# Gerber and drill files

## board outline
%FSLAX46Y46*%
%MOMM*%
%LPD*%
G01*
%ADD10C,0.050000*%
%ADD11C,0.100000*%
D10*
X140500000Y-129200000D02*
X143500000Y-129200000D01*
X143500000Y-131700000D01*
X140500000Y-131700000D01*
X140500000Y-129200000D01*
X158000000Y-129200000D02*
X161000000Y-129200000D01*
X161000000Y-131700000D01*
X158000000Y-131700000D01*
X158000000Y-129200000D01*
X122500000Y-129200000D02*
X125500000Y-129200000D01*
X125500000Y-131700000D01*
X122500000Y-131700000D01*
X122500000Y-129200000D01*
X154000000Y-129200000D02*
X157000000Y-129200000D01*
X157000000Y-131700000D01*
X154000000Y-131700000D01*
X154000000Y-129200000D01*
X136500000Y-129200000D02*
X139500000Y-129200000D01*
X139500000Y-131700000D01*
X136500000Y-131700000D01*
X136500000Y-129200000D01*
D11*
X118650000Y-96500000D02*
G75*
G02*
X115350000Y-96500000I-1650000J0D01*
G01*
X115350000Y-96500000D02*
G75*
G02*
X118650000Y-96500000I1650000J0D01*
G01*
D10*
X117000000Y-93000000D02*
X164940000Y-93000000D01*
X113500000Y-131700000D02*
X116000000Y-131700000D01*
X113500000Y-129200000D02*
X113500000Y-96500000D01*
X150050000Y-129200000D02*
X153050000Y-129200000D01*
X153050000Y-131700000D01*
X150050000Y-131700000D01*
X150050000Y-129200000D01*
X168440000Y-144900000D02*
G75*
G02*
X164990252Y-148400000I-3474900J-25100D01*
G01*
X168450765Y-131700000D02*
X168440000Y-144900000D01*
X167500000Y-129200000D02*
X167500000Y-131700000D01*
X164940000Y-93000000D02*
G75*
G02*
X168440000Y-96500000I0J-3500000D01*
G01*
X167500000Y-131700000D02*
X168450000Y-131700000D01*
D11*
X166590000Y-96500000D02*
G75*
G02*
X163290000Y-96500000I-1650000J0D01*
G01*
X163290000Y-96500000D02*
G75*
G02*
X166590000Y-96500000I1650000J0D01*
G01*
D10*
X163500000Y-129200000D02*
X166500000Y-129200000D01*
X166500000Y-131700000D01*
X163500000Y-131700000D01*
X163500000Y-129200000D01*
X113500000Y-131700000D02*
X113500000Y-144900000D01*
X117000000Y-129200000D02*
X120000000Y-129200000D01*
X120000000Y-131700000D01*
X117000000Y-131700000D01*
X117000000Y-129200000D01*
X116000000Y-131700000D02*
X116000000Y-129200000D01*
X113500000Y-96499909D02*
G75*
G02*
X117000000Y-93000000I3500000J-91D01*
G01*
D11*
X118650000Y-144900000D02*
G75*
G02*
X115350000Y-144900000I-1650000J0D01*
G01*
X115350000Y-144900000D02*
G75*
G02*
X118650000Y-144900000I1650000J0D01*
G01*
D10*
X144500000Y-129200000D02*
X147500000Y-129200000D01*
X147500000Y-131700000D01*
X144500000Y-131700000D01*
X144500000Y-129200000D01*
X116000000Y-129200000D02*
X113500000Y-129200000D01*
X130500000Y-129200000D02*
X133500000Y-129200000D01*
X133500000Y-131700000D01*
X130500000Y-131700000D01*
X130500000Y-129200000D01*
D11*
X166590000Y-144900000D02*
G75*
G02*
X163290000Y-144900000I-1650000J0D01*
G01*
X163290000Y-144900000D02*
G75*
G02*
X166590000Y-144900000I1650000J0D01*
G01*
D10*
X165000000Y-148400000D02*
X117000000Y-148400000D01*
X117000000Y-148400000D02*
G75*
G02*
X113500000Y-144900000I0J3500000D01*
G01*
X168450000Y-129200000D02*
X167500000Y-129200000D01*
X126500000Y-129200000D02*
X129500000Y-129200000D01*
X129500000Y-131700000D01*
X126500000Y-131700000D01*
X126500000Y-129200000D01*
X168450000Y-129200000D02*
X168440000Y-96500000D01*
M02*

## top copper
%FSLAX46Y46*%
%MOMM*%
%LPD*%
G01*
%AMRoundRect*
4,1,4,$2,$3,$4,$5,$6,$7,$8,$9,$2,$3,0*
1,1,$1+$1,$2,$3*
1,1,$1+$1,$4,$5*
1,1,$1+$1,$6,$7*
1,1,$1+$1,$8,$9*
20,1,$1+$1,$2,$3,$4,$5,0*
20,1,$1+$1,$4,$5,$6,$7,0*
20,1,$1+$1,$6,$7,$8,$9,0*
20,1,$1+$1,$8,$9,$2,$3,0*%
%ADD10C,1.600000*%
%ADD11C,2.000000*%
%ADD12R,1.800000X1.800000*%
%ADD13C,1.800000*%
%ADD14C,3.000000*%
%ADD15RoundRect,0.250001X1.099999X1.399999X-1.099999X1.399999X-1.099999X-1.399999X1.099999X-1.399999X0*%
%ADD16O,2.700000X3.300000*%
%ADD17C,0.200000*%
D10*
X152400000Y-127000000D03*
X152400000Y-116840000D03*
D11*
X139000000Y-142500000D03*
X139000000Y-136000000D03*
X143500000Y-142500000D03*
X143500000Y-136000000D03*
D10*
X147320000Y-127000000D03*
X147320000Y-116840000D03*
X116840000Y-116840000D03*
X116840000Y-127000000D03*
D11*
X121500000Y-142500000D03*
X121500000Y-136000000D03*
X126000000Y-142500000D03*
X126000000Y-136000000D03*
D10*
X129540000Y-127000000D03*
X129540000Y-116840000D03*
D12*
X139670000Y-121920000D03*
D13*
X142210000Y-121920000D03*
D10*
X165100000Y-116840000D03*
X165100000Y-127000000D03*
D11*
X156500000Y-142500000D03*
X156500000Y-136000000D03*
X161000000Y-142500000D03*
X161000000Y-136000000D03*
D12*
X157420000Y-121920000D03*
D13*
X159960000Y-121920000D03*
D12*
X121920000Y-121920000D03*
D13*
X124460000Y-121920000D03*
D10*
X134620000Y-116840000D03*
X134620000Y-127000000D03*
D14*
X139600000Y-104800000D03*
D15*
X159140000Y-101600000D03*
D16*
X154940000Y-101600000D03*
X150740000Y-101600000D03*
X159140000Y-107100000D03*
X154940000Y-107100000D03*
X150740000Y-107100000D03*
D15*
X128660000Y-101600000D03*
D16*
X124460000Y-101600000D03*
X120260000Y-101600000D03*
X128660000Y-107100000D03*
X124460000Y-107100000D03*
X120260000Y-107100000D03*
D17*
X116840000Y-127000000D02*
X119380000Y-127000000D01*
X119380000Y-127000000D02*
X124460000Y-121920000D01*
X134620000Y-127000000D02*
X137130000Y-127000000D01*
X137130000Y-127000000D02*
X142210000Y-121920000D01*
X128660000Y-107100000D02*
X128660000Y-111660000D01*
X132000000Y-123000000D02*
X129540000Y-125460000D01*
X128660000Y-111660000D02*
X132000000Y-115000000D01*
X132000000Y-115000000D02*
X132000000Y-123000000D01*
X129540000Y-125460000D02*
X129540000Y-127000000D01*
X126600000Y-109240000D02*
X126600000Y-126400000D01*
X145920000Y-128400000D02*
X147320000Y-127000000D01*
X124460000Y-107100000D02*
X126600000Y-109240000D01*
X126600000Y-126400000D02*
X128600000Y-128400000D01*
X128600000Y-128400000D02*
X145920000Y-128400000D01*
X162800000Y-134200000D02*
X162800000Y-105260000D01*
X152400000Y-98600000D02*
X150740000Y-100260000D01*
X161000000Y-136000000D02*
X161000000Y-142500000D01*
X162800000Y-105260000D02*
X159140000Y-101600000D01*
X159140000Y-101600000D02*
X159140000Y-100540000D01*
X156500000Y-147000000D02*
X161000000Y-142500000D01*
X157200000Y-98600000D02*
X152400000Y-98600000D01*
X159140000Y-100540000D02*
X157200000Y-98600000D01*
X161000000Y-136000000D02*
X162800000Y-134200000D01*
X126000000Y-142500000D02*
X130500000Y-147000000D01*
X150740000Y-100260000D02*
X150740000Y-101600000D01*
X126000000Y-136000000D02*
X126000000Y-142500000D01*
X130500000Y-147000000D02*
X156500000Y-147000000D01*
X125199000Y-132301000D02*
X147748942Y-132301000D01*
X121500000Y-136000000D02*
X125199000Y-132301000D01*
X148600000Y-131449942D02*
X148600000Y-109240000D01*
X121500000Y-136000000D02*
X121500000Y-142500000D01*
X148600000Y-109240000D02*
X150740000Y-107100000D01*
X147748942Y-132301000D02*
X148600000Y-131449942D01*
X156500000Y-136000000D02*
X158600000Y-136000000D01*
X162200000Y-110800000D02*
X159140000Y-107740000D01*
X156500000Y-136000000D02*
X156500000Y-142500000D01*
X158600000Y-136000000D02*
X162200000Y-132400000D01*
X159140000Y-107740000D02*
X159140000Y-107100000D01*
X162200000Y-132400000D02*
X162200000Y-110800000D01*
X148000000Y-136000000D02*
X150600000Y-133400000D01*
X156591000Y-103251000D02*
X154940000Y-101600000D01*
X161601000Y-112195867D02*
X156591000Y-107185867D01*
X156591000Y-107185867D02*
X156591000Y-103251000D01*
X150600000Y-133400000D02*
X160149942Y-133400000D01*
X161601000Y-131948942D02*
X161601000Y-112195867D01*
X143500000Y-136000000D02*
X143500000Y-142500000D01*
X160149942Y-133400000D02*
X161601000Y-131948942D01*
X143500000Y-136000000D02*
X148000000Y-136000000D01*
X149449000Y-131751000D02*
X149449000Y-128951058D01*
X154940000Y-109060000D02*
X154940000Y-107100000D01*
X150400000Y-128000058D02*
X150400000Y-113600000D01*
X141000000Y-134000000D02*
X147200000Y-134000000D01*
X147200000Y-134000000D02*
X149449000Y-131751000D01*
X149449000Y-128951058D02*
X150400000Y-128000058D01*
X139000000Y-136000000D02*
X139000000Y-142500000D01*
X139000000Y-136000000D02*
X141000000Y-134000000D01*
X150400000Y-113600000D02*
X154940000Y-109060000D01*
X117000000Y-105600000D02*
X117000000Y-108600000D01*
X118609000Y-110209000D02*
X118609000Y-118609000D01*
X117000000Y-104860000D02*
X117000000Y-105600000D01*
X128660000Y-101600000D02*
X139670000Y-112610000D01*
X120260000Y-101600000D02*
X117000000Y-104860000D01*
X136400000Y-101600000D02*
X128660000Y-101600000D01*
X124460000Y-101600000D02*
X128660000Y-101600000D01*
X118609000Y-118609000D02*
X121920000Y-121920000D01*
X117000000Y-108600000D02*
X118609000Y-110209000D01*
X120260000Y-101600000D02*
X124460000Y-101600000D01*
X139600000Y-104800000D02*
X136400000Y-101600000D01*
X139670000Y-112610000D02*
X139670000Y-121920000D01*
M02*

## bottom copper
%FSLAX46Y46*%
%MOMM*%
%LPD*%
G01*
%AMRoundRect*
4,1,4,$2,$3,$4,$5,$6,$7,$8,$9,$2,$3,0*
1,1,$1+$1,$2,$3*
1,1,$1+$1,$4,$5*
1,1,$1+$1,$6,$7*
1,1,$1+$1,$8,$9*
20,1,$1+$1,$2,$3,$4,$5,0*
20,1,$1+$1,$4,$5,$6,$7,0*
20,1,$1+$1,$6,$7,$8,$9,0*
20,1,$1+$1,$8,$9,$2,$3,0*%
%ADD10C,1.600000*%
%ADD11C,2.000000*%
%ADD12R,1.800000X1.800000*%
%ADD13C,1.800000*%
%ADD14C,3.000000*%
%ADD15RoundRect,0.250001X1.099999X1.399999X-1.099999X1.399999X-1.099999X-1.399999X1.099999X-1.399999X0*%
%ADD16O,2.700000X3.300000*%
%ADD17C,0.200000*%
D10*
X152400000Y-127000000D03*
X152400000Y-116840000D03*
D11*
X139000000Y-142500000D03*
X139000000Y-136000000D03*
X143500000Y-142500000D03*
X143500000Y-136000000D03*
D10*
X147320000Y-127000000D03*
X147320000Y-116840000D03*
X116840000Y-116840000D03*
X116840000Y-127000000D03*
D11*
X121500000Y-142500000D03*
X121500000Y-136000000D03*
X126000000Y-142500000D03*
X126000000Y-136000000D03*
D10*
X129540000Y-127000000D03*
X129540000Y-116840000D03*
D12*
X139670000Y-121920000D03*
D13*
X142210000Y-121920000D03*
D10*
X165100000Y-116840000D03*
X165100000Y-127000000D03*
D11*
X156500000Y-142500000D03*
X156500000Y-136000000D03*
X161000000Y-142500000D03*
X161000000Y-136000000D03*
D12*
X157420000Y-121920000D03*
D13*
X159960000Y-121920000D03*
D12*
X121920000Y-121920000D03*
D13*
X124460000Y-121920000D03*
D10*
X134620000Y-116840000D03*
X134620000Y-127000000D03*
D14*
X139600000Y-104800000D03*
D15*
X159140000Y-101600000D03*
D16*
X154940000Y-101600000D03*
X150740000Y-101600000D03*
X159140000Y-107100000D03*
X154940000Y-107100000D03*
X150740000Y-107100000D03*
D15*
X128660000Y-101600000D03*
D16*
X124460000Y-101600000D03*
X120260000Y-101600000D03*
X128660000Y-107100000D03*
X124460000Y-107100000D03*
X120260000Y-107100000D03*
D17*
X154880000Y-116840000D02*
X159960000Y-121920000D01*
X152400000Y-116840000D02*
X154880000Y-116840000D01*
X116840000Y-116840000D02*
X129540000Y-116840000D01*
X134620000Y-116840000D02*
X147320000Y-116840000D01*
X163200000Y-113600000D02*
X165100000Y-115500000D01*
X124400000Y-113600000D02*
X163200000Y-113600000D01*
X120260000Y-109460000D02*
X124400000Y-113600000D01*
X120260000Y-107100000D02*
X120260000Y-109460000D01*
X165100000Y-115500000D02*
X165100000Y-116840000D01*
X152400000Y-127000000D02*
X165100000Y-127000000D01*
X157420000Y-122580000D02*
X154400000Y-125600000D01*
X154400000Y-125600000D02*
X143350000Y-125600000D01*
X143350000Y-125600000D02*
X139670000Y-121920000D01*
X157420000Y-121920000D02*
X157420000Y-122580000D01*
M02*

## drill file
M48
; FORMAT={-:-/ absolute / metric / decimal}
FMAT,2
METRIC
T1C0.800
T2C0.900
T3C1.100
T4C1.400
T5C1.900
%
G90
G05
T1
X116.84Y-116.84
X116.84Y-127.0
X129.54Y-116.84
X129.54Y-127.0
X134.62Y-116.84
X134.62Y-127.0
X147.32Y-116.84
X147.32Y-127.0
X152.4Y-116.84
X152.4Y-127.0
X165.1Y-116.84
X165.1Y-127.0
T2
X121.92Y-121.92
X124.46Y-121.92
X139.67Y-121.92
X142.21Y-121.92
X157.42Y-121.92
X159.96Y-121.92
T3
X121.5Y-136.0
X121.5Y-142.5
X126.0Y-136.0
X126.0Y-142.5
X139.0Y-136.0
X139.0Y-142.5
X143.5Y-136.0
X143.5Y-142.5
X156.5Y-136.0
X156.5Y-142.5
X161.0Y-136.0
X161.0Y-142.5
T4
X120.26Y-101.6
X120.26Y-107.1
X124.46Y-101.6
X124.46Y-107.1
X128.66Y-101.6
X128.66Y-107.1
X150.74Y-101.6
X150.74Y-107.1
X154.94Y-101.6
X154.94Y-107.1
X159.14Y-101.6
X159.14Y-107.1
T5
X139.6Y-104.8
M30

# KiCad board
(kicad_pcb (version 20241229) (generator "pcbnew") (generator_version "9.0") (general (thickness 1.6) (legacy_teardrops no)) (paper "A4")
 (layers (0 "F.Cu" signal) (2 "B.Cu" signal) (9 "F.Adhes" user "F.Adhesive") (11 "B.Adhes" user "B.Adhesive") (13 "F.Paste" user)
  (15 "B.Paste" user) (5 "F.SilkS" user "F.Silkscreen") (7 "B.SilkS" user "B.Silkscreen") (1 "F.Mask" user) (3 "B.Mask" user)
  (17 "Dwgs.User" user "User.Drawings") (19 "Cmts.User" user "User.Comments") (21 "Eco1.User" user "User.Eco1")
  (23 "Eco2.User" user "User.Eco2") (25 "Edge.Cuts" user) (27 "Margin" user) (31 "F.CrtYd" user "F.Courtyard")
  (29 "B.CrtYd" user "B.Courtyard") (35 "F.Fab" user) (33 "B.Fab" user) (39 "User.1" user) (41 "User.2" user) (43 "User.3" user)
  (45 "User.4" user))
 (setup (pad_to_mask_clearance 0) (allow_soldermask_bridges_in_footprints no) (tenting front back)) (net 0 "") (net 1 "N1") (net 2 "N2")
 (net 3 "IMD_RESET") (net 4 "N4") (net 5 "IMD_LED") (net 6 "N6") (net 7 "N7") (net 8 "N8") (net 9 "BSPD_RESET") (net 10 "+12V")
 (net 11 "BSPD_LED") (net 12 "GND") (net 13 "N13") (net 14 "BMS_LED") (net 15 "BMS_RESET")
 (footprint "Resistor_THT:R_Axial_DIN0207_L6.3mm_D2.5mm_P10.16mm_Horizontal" (layer "F.Cu") (at 152.4 127 90)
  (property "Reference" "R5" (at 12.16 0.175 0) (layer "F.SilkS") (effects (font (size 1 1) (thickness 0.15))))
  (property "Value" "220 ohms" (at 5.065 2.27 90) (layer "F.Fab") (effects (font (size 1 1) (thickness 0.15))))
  (pad "1" thru_hole circle (at 0 0 90) (size 1.6 1.6) (drill 0.8) (layers "*.Cu" "*.Mask") (remove_unused_layers no) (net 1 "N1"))
  (pad "2" thru_hole circle (at 10.16 0 90) (size 1.6 1.6) (drill 0.8) (layers "*.Cu" "*.Mask") (remove_unused_layers no) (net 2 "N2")))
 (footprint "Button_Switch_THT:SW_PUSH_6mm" (layer "F.Cu") (at 139 142.5 90)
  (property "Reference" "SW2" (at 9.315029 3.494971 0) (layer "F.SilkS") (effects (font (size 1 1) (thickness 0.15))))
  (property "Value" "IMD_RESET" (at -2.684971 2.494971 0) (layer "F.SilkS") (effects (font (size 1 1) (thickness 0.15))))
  (pad "1" thru_hole circle (at 0 0 180) (size 2 2) (drill 1.1) (layers "*.Cu" "*.Mask") (remove_unused_layers no) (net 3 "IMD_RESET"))
  (pad "1" thru_hole circle (at 6.5 0 180) (size 2 2) (drill 1.1) (layers "*.Cu" "*.Mask") (remove_unused_layers no) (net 3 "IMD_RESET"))
  (pad "2" thru_hole circle (at 0 4.5 180) (size 2 2) (drill 1.1) (layers "*.Cu" "*.Mask") (remove_unused_layers no) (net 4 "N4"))
  (pad "2" thru_hole circle (at 6.5 4.5 180) (size 2 2) (drill 1.1) (layers "*.Cu" "*.Mask") (remove_unused_layers no) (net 4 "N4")))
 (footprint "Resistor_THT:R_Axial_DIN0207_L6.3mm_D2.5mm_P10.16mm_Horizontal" (layer "F.Cu") (at 147.32 127 90)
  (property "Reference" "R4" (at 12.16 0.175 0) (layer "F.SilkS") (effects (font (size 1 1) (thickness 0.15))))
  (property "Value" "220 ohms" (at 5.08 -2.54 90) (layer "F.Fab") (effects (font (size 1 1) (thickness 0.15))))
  (pad "1" thru_hole circle (at 0 0 90) (size 1.6 1.6) (drill 0.8) (layers "*.Cu" "*.Mask") (remove_unused_layers no) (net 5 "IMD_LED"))
  (pad "2" thru_hole circle (at 10.16 0 90) (size 1.6 1.6) (drill 0.8) (layers "*.Cu" "*.Mask") (remove_unused_layers no) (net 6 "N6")))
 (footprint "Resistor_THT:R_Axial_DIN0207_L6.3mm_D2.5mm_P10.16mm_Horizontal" (layer "F.Cu") (at 116.84 116.84 -90)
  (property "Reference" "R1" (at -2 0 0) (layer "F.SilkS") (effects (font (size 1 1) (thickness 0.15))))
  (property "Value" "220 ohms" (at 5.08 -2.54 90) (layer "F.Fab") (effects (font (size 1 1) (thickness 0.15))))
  (pad "1" thru_hole circle (at 0 0 270) (size 1.6 1.6) (drill 0.8) (layers "*.Cu" "*.Mask") (remove_unused_layers no) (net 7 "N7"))
  (pad "2" thru_hole circle (at 10.16 0 270) (size 1.6 1.6) (drill 0.8) (layers "*.Cu" "*.Mask") (remove_unused_layers no) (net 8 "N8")))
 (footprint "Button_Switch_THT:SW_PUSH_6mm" (layer "F.Cu") (at 121.5 142.5 90)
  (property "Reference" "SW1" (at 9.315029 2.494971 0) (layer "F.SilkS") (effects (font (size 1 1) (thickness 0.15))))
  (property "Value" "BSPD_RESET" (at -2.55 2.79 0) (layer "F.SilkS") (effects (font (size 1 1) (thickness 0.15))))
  (pad "1" thru_hole circle (at 0 0 180) (size 2 2) (drill 1.1) (layers "*.Cu" "*.Mask") (remove_unused_layers no) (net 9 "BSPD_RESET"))
  (pad "1" thru_hole circle (at 6.5 0 180) (size 2 2) (drill 1.1) (layers "*.Cu" "*.Mask") (remove_unused_layers no) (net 9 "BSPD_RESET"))
  (pad "2" thru_hole circle (at 0 4.5 180) (size 2 2) (drill 1.1) (layers "*.Cu" "*.Mask") (remove_unused_layers no) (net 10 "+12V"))
  (pad "2" thru_hole circle (at 6.5 4.5 180) (size 2 2) (drill 1.1) (layers "*.Cu" "*.Mask") (remove_unused_layers no) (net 10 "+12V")))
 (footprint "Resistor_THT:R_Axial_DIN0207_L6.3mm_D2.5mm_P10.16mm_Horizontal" (layer "F.Cu") (at 129.54 127 90)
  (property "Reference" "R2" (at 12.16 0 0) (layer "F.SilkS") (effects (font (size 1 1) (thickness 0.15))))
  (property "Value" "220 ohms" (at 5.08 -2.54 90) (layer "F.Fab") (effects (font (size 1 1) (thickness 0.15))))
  (pad "1" thru_hole circle (at 0 0 90) (size 1.6 1.6) (drill 0.8) (layers "*.Cu" "*.Mask") (remove_unused_layers no) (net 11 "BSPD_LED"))
  (pad "2" thru_hole circle (at 10.16 0 90) (size 1.6 1.6) (drill 0.8) (layers "*.Cu" "*.Mask") (remove_unused_layers no) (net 7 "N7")))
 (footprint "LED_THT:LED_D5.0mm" (layer "F.Cu") (at 139.67 121.92)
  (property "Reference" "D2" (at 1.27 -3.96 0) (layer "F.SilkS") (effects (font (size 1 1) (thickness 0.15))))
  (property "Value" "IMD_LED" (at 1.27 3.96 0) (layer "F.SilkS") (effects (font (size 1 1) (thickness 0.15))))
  (pad "1" thru_hole rect (at 0 0) (size 1.8 1.8) (drill 0.9) (layers "*.Cu" "*.Mask") (remove_unused_layers no) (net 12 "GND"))
  (pad "2" thru_hole circle (at 2.54 0) (size 1.8 1.8) (drill 0.9) (layers "*.Cu" "*.Mask") (remove_unused_layers no) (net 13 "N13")))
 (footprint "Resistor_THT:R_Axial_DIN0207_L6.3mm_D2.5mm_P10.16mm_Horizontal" (layer "F.Cu") (at 165.1 116.84 -90)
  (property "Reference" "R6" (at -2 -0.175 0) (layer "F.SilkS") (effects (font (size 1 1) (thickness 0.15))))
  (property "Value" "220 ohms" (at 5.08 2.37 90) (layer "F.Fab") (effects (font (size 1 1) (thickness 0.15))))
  (pad "1" thru_hole circle (at 0 0 270) (size 1.6 1.6) (drill 0.8) (layers "*.Cu" "*.Mask") (remove_unused_layers no) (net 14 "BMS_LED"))
  (pad "2" thru_hole circle (at 10.16 0 270) (size 1.6 1.6) (drill 0.8) (layers "*.Cu" "*.Mask") (remove_unused_layers no) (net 1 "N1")))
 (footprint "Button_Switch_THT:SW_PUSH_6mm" (layer "F.Cu") (at 156.5 142.5 90)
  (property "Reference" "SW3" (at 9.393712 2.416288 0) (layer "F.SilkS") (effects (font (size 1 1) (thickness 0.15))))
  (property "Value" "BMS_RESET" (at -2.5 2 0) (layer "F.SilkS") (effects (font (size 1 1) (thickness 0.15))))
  (pad "1" thru_hole circle (at 0 0 180) (size 2 2) (drill 1.1) (layers "*.Cu" "*.Mask") (remove_unused_layers no) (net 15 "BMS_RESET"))
  (pad "1" thru_hole circle (at 6.5 0 180) (size 2 2) (drill 1.1) (layers "*.Cu" "*.Mask") (remove_unused_layers no) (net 15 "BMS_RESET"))
  (pad "2" thru_hole circle (at 0 4.5 180) (size 2 2) (drill 1.1) (layers "*.Cu" "*.Mask") (remove_unused_layers no) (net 10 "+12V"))
  (pad "2" thru_hole circle (at 6.5 4.5 180) (size 2 2) (drill 1.1) (layers "*.Cu" "*.Mask") (remove_unused_layers no) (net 10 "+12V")))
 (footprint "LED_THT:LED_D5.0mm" (layer "F.Cu") (at 157.42 121.92)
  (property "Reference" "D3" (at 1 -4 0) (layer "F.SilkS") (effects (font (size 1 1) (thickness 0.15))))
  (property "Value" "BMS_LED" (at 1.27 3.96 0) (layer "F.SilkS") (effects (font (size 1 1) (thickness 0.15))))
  (pad "1" thru_hole rect (at 0 0) (size 1.8 1.8) (drill 0.9) (layers "*.Cu" "*.Mask") (remove_unused_layers no) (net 12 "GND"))
  (pad "2" thru_hole circle (at 2.54 0) (size 1.8 1.8) (drill 0.9) (layers "*.Cu" "*.Mask") (remove_unused_layers no) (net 2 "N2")))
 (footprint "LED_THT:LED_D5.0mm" (layer "F.Cu") (at 121.92 121.92)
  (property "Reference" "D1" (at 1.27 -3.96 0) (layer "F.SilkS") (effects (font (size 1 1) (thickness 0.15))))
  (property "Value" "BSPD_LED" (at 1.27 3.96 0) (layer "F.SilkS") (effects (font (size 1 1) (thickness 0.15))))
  (pad "1" thru_hole rect (at 0 0) (size 1.8 1.8) (drill 0.9) (layers "*.Cu" "*.Mask") (remove_unused_layers no) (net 12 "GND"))
  (pad "2" thru_hole circle (at 2.54 0) (size 1.8 1.8) (drill 0.9) (layers "*.Cu" "*.Mask") (remove_unused_layers no) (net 8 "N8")))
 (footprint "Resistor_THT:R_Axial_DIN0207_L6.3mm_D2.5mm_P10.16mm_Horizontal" (layer "F.Cu") (at 134.62 116.84 -90)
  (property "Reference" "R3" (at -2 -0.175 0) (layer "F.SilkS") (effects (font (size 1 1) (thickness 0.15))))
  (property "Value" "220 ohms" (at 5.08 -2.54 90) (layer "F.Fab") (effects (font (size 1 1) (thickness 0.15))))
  (pad "1" thru_hole circle (at 0 0 270) (size 1.6 1.6) (drill 0.8) (layers "*.Cu" "*.Mask") (remove_unused_layers no) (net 6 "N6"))
  (pad "2" thru_hole circle (at 10.16 0 270) (size 1.6 1.6) (drill 0.8) (layers "*.Cu" "*.Mask") (remove_unused_layers no) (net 13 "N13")))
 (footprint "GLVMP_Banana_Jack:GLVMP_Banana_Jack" (layer "B.Cu") (at 139.6 104.8 180)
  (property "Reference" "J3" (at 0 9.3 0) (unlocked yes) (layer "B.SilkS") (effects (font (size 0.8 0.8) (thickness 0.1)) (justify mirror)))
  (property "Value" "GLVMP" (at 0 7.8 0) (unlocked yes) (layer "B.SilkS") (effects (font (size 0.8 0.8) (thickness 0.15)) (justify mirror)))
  (pad "1" thru_hole circle (at 0 0 180) (size 3 3) (drill 1.9) (layers "*.Cu" "*.Mask") (remove_unused_layers no) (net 12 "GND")))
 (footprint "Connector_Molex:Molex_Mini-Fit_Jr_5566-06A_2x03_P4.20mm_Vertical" (layer "B.Cu") (at 159.14 101.6 180)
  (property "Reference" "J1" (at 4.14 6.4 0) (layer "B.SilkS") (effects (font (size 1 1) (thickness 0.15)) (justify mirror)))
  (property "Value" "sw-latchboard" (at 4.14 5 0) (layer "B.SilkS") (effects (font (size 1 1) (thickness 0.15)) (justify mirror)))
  (pad "1" thru_hole roundrect (at 0 0 180) (size 2.7 3.3) (drill 1.4) (layers "*.Cu" "*.Mask") (remove_unused_layers no)
   (roundrect_rratio 0.092593) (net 10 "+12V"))
  (pad "2" thru_hole oval (at 4.2 0 180) (size 2.7 3.3) (drill 1.4) (layers "*.Cu" "*.Mask") (remove_unused_layers no) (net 4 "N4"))
  (pad "3" thru_hole oval (at 8.4 0 180) (size 2.7 3.3) (drill 1.4) (layers "*.Cu" "*.Mask") (remove_unused_layers no) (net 10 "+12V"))
  (pad "4" thru_hole oval (at 0 -5.5 180) (size 2.7 3.3) (drill 1.4) (layers "*.Cu" "*.Mask") (remove_unused_layers no) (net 15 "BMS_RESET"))
  (pad "5" thru_hole oval (at 4.2 -5.5 180) (size 2.7 3.3) (drill 1.4) (layers "*.Cu" "*.Mask") (remove_unused_layers no)
   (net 3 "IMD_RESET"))
  (pad "6" thru_hole oval (at 8.4 -5.5 180) (size 2.7 3.3) (drill 1.4) (layers "*.Cu" "*.Mask") (remove_unused_layers no)
   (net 9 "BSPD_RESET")))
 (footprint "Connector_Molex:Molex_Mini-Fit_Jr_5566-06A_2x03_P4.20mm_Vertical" (layer "B.Cu") (at 128.66 101.6 180)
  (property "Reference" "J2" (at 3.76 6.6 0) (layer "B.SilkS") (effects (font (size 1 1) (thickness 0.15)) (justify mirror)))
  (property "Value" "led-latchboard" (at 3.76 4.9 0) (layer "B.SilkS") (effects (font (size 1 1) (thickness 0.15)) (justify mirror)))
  (pad "1" thru_hole roundrect (at 0 0 180) (size 2.7 3.3) (drill 1.4) (layers "*.Cu" "*.Mask") (remove_unused_layers no)
   (roundrect_rratio 0.092593) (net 12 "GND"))
  (pad "2" thru_hole oval (at 4.2 0 180) (size 2.7 3.3) (drill 1.4) (layers "*.Cu" "*.Mask") (remove_unused_layers no) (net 12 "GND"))
  (pad "3" thru_hole oval (at 8.4 0 180) (size 2.7 3.3) (drill 1.4) (layers "*.Cu" "*.Mask") (remove_unused_layers no) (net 12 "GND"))
  (pad "4" thru_hole oval (at 0 -5.5 180) (size 2.7 3.3) (drill 1.4) (layers "*.Cu" "*.Mask") (remove_unused_layers no) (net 11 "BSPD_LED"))
  (pad "5" thru_hole oval (at 4.2 -5.5 180) (size 2.7 3.3) (drill 1.4) (layers "*.Cu" "*.Mask") (remove_unused_layers no) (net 5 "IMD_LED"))
  (pad "6" thru_hole oval (at 8.4 -5.5 180) (size 2.7 3.3) (drill 1.4) (layers "*.Cu" "*.Mask") (remove_unused_layers no) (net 14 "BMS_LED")))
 (gr_rect (start 140.5 129.2) (end 143.5 131.7) (stroke (width 0.05) (type default)) (fill no) (layer "Edge.Cuts"))
 (gr_rect (start 158 129.2) (end 161 131.7) (stroke (width 0.05) (type default)) (fill no) (layer "Edge.Cuts"))
 (gr_rect (start 122.5 129.2) (end 125.5 131.7) (stroke (width 0.05) (type default)) (fill no) (layer "Edge.Cuts"))
 (gr_rect (start 154 129.2) (end 157 131.7) (stroke (width 0.05) (type default)) (fill no) (layer "Edge.Cuts"))
 (gr_rect (start 136.5 129.2) (end 139.5 131.7) (stroke (width 0.05) (type default)) (fill no) (layer "Edge.Cuts"))
 (gr_circle (center 117 96.5) (end 118.65 96.5) (stroke (width 0.1) (type solid)) (fill no) (layer "Edge.Cuts"))
 (gr_line (start 117 93) (end 164.94 93) (stroke (width 0.05) (type default)) (layer "Edge.Cuts"))
 (gr_line (start 113.5 131.7) (end 116 131.7) (stroke (width 0.05) (type default)) (layer "Edge.Cuts"))
 (gr_line (start 113.5 129.2) (end 113.5 96.5) (stroke (width 0.05) (type default)) (layer "Edge.Cuts"))
 (gr_rect (start 150.05 129.2) (end 153.05 131.7) (stroke (width 0.05) (type default)) (fill no) (layer "Edge.Cuts"))
 (gr_arc (start 168.44 144.9) (mid 167.44 147.364466) (end 164.990252 148.4) (stroke (width 0.05) (type solid)) (layer "Edge.Cuts"))
 (gr_line (start 168.450765 131.7) (end 168.44 144.9) (stroke (width 0.05) (type default)) (layer "Edge.Cuts"))
 (gr_line (start 167.5 129.2) (end 167.5 131.7) (stroke (width 0.05) (type default)) (layer "Edge.Cuts"))
 (gr_arc (start 164.94 93) (mid 167.414874 94.025126) (end 168.44 96.5) (stroke (width 0.05) (type solid)) (layer "Edge.Cuts"))
 (gr_line (start 167.5 131.7) (end 168.45 131.7) (stroke (width 0.05) (type default)) (layer "Edge.Cuts"))
 (gr_circle (center 164.94 96.5) (end 166.59 96.5) (stroke (width 0.1) (type solid)) (fill no) (layer "Edge.Cuts"))
 (gr_rect (start 163.5 129.2) (end 166.5 131.7) (stroke (width 0.05) (type default)) (fill no) (layer "Edge.Cuts"))
 (gr_line (start 113.5 131.7) (end 113.5 144.9) (stroke (width 0.05) (type solid)) (layer "Edge.Cuts"))
 (gr_rect (start 117 129.2) (end 120 131.7) (stroke (width 0.05) (type default)) (fill no) (layer "Edge.Cuts"))
 (gr_line (start 116 131.7) (end 116 129.2) (stroke (width 0.05) (type default)) (layer "Edge.Cuts"))
 (gr_arc (start 113.5 96.499909) (mid 114.525158 94.025094) (end 117 93) (stroke (width 0.05) (type default)) (layer "Edge.Cuts"))
 (gr_circle (center 117 144.9) (end 115.35 144.9) (stroke (width 0.1) (type solid)) (fill no) (layer "Edge.Cuts"))
 (gr_rect (start 144.5 129.2) (end 147.5 131.7) (stroke (width 0.05) (type default)) (fill no) (layer "Edge.Cuts"))
 (gr_line (start 116 129.2) (end 113.5 129.2) (stroke (width 0.05) (type default)) (layer "Edge.Cuts"))
 (gr_rect (start 130.5 129.2) (end 133.5 131.7) (stroke (width 0.05) (type default)) (fill no) (layer "Edge.Cuts"))
 (gr_circle (center 164.94 144.9) (end 163.29 144.9) (stroke (width 0.1) (type solid)) (fill no) (layer "Edge.Cuts"))
 (gr_line (start 165 148.4) (end 117 148.4) (stroke (width 0.05) (type solid)) (layer "Edge.Cuts"))
 (gr_arc (start 117 148.4) (mid 114.525126 147.374874) (end 113.5 144.9) (stroke (width 0.05) (type solid)) (layer "Edge.Cuts"))
 (gr_line (start 168.45 129.2) (end 167.5 129.2) (stroke (width 0.05) (type default)) (layer "Edge.Cuts"))
 (gr_rect (start 126.5 129.2) (end 129.5 131.7) (stroke (width 0.05) (type default)) (fill no) (layer "Edge.Cuts"))
 (gr_line (start 168.45 129.2) (end 168.44 96.5) (stroke (width 0.05) (type default)) (layer "Edge.Cuts"))
 (segment (start 116.84 127) (end 119.38 127) (width 0.2) (layer "F.Cu") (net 8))
 (segment (start 119.38 127) (end 124.46 121.92) (width 0.2) (layer "F.Cu") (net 8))
 (segment (start 134.62 127) (end 137.13 127) (width 0.2) (layer "F.Cu") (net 13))
 (segment (start 137.13 127) (end 142.21 121.92) (width 0.2) (layer "F.Cu") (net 13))
 (segment (start 154.88 116.84) (end 159.96 121.92) (width 0.2) (layer "B.Cu") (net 2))
 (segment (start 152.4 116.84) (end 154.88 116.84) (width 0.2) (layer "B.Cu") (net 2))
 (segment (start 116.84 116.84) (end 129.54 116.84) (width 0.2) (layer "B.Cu") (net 7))
 (segment (start 128.66 107.1) (end 128.66 111.66) (width 0.2) (layer "F.Cu") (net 11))
 (segment (start 132 123) (end 129.54 125.46) (width 0.2) (layer "F.Cu") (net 11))
 (segment (start 128.66 111.66) (end 132 115) (width 0.2) (layer "F.Cu") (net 11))
 (segment (start 132 115) (end 132 123) (width 0.2) (layer "F.Cu") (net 11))
 (segment (start 129.54 125.46) (end 129.54 127) (width 0.2) (layer "F.Cu") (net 11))
 (segment (start 134.62 116.84) (end 147.32 116.84) (width 0.2) (layer "B.Cu") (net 6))
 (segment (start 126.6 109.24) (end 126.6 126.4) (width 0.2) (layer "F.Cu") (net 5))
 (segment (start 145.92 128.4) (end 147.32 127) (width 0.2) (layer "F.Cu") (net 5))
 (segment (start 124.46 107.1) (end 126.6 109.24) (width 0.2) (layer "F.Cu") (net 5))
 (segment (start 126.6 126.4) (end 128.6 128.4) (width 0.2) (layer "F.Cu") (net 5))
 (segment (start 128.6 128.4) (end 145.92 128.4) (width 0.2) (layer "F.Cu") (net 5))
 (segment (start 163.2 113.6) (end 165.1 115.5) (width 0.2) (layer "B.Cu") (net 14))
 (segment (start 124.4 113.6) (end 163.2 113.6) (width 0.2) (layer "B.Cu") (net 14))
 (segment (start 120.26 109.46) (end 124.4 113.6) (width 0.2) (layer "B.Cu") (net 14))
 (segment (start 120.26 107.1) (end 120.26 109.46) (width 0.2) (layer "B.Cu") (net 14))
 (segment (start 165.1 115.5) (end 165.1 116.84) (width 0.2) (layer "B.Cu") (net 14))
 (segment (start 162.8 134.2) (end 162.8 105.26) (width 0.2) (layer "F.Cu") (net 10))
 (segment (start 152.4 98.6) (end 150.74 100.26) (width 0.2) (layer "F.Cu") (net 10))
 (segment (start 161 136) (end 161 142.5) (width 0.2) (layer "F.Cu") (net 10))
 (segment (start 162.8 105.26) (end 159.14 101.6) (width 0.2) (layer "F.Cu") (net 10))
 (segment (start 159.14 101.6) (end 159.14 100.54) (width 0.2) (layer "F.Cu") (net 10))
 (segment (start 156.5 147) (end 161 142.5) (width 0.2) (layer "F.Cu") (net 10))
 (segment (start 157.2 98.6) (end 152.4 98.6) (width 0.2) (layer "F.Cu") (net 10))
 (segment (start 159.14 100.54) (end 157.2 98.6) (width 0.2) (layer "F.Cu") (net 10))
 (segment (start 161 136) (end 162.8 134.2) (width 0.2) (layer "F.Cu") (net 10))
 (segment (start 126 142.5) (end 130.5 147) (width 0.2) (layer "F.Cu") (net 10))
 (segment (start 150.74 100.26) (end 150.74 101.6) (width 0.2) (layer "F.Cu") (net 10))
 (segment (start 126 136) (end 126 142.5) (width 0.2) (layer "F.Cu") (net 10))
 (segment (start 130.5 147) (end 156.5 147) (width 0.2) (layer "F.Cu") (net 10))
 (segment (start 125.199 132.301) (end 147.748942 132.301) (width 0.2) (layer "F.Cu") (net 9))
 (segment (start 121.5 136) (end 125.199 132.301) (width 0.2) (layer "F.Cu") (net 9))
 (segment (start 148.6 131.449942) (end 148.6 109.24) (width 0.2) (layer "F.Cu") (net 9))
 (segment (start 121.5 136) (end 121.5 142.5) (width 0.2) (layer "F.Cu") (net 9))
 (segment (start 148.6 109.24) (end 150.74 107.1) (width 0.2) (layer "F.Cu") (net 9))
 (segment (start 147.748942 132.301) (end 148.6 131.449942) (width 0.2) (layer "F.Cu") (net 9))
 (segment (start 156.5 136) (end 158.6 136) (width 0.2) (layer "F.Cu") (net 15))
 (segment (start 162.2 110.8) (end 159.14 107.74) (width 0.2) (layer "F.Cu") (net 15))
 (segment (start 156.5 136) (end 156.5 142.5) (width 0.2) (layer "F.Cu") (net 15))
 (segment (start 158.6 136) (end 162.2 132.4) (width 0.2) (layer "F.Cu") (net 15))
 (segment (start 159.14 107.74) (end 159.14 107.1) (width 0.2) (layer "F.Cu") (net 15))
 (segment (start 162.2 132.4) (end 162.2 110.8) (width 0.2) (layer "F.Cu") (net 15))
 (segment (start 148 136) (end 150.6 133.4) (width 0.2) (layer "F.Cu") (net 4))
 (segment (start 156.591 103.251) (end 154.94 101.6) (width 0.2) (layer "F.Cu") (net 4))
 (segment (start 161.601 112.195867) (end 156.591 107.185867) (width 0.2) (layer "F.Cu") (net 4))
 (segment (start 156.591 107.185867) (end 156.591 103.251) (width 0.2) (layer "F.Cu") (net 4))
 (segment (start 150.6 133.4) (end 160.149942 133.4) (width 0.2) (layer "F.Cu") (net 4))
 (segment (start 161.601 131.948942) (end 161.601 112.195867) (width 0.2) (layer "F.Cu") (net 4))
 (segment (start 143.5 136) (end 143.5 142.5) (width 0.2) (layer "F.Cu") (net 4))
 (segment (start 160.149942 133.4) (end 161.601 131.948942) (width 0.2) (layer "F.Cu") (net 4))
 (segment (start 143.5 136) (end 148 136) (width 0.2) (layer "F.Cu") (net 4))
 (segment (start 149.449 131.751) (end 149.449 128.951058) (width 0.2) (layer "F.Cu") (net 3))
 (segment (start 154.94 109.06) (end 154.94 107.1) (width 0.2) (layer "F.Cu") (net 3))
 (segment (start 150.4 128.000058) (end 150.4 113.6) (width 0.2) (layer "F.Cu") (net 3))
 (segment (start 141 134) (end 147.2 134) (width 0.2) (layer "F.Cu") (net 3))
 (segment (start 147.2 134) (end 149.449 131.751) (width 0.2) (layer "F.Cu") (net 3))
 (segment (start 149.449 128.951058) (end 150.4 128.000058) (width 0.2) (layer "F.Cu") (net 3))
 (segment (start 139 136) (end 139 142.5) (width 0.2) (layer "F.Cu") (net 3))
 (segment (start 139 136) (end 141 134) (width 0.2) (layer "F.Cu") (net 3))
 (segment (start 150.4 113.6) (end 154.94 109.06) (width 0.2) (layer "F.Cu") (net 3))
 (segment (start 152.4 127) (end 165.1 127) (width 0.2) (layer "B.Cu") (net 1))
 (segment (start 117 105.6) (end 117 108.6) (width 0.2) (layer "F.Cu") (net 12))
 (segment (start 118.609 110.209) (end 118.609 118.609) (width 0.2) (layer "F.Cu") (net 12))
 (segment (start 117 104.86) (end 117 105.6) (width 0.2) (layer "F.Cu") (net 12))
 (segment (start 128.66 101.6) (end 139.67 112.61) (width 0.2) (layer "F.Cu") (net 12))
 (segment (start 120.26 101.6) (end 117 104.86) (width 0.2) (layer "F.Cu") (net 12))
 (segment (start 136.4 101.6) (end 128.66 101.6) (width 0.2) (layer "F.Cu") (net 12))
 (segment (start 124.46 101.6) (end 128.66 101.6) (width 0.2) (layer "F.Cu") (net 12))
 (segment (start 118.609 118.609) (end 121.92 121.92) (width 0.2) (layer "F.Cu") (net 12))
 (segment (start 117 108.6) (end 118.609 110.209) (width 0.2) (layer "F.Cu") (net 12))
 (segment (start 120.26 101.6) (end 124.46 101.6) (width 0.2) (layer "F.Cu") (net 12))
 (segment (start 139.6 104.8) (end 136.4 101.6) (width 0.2) (layer "F.Cu") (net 12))
 (segment (start 139.67 112.61) (end 139.67 121.92) (width 0.2) (layer "F.Cu") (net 12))
 (segment (start 157.42 122.58) (end 154.4 125.6) (width 0.2) (layer "B.Cu") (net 12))
 (segment (start 154.4 125.6) (end 143.35 125.6) (width 0.2) (layer "B.Cu") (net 12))
 (segment (start 143.35 125.6) (end 139.67 121.92) (width 0.2) (layer "B.Cu") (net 12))
 (segment (start 157.42 121.92) (end 157.42 122.58) (width 0.2) (layer "B.Cu") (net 12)))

